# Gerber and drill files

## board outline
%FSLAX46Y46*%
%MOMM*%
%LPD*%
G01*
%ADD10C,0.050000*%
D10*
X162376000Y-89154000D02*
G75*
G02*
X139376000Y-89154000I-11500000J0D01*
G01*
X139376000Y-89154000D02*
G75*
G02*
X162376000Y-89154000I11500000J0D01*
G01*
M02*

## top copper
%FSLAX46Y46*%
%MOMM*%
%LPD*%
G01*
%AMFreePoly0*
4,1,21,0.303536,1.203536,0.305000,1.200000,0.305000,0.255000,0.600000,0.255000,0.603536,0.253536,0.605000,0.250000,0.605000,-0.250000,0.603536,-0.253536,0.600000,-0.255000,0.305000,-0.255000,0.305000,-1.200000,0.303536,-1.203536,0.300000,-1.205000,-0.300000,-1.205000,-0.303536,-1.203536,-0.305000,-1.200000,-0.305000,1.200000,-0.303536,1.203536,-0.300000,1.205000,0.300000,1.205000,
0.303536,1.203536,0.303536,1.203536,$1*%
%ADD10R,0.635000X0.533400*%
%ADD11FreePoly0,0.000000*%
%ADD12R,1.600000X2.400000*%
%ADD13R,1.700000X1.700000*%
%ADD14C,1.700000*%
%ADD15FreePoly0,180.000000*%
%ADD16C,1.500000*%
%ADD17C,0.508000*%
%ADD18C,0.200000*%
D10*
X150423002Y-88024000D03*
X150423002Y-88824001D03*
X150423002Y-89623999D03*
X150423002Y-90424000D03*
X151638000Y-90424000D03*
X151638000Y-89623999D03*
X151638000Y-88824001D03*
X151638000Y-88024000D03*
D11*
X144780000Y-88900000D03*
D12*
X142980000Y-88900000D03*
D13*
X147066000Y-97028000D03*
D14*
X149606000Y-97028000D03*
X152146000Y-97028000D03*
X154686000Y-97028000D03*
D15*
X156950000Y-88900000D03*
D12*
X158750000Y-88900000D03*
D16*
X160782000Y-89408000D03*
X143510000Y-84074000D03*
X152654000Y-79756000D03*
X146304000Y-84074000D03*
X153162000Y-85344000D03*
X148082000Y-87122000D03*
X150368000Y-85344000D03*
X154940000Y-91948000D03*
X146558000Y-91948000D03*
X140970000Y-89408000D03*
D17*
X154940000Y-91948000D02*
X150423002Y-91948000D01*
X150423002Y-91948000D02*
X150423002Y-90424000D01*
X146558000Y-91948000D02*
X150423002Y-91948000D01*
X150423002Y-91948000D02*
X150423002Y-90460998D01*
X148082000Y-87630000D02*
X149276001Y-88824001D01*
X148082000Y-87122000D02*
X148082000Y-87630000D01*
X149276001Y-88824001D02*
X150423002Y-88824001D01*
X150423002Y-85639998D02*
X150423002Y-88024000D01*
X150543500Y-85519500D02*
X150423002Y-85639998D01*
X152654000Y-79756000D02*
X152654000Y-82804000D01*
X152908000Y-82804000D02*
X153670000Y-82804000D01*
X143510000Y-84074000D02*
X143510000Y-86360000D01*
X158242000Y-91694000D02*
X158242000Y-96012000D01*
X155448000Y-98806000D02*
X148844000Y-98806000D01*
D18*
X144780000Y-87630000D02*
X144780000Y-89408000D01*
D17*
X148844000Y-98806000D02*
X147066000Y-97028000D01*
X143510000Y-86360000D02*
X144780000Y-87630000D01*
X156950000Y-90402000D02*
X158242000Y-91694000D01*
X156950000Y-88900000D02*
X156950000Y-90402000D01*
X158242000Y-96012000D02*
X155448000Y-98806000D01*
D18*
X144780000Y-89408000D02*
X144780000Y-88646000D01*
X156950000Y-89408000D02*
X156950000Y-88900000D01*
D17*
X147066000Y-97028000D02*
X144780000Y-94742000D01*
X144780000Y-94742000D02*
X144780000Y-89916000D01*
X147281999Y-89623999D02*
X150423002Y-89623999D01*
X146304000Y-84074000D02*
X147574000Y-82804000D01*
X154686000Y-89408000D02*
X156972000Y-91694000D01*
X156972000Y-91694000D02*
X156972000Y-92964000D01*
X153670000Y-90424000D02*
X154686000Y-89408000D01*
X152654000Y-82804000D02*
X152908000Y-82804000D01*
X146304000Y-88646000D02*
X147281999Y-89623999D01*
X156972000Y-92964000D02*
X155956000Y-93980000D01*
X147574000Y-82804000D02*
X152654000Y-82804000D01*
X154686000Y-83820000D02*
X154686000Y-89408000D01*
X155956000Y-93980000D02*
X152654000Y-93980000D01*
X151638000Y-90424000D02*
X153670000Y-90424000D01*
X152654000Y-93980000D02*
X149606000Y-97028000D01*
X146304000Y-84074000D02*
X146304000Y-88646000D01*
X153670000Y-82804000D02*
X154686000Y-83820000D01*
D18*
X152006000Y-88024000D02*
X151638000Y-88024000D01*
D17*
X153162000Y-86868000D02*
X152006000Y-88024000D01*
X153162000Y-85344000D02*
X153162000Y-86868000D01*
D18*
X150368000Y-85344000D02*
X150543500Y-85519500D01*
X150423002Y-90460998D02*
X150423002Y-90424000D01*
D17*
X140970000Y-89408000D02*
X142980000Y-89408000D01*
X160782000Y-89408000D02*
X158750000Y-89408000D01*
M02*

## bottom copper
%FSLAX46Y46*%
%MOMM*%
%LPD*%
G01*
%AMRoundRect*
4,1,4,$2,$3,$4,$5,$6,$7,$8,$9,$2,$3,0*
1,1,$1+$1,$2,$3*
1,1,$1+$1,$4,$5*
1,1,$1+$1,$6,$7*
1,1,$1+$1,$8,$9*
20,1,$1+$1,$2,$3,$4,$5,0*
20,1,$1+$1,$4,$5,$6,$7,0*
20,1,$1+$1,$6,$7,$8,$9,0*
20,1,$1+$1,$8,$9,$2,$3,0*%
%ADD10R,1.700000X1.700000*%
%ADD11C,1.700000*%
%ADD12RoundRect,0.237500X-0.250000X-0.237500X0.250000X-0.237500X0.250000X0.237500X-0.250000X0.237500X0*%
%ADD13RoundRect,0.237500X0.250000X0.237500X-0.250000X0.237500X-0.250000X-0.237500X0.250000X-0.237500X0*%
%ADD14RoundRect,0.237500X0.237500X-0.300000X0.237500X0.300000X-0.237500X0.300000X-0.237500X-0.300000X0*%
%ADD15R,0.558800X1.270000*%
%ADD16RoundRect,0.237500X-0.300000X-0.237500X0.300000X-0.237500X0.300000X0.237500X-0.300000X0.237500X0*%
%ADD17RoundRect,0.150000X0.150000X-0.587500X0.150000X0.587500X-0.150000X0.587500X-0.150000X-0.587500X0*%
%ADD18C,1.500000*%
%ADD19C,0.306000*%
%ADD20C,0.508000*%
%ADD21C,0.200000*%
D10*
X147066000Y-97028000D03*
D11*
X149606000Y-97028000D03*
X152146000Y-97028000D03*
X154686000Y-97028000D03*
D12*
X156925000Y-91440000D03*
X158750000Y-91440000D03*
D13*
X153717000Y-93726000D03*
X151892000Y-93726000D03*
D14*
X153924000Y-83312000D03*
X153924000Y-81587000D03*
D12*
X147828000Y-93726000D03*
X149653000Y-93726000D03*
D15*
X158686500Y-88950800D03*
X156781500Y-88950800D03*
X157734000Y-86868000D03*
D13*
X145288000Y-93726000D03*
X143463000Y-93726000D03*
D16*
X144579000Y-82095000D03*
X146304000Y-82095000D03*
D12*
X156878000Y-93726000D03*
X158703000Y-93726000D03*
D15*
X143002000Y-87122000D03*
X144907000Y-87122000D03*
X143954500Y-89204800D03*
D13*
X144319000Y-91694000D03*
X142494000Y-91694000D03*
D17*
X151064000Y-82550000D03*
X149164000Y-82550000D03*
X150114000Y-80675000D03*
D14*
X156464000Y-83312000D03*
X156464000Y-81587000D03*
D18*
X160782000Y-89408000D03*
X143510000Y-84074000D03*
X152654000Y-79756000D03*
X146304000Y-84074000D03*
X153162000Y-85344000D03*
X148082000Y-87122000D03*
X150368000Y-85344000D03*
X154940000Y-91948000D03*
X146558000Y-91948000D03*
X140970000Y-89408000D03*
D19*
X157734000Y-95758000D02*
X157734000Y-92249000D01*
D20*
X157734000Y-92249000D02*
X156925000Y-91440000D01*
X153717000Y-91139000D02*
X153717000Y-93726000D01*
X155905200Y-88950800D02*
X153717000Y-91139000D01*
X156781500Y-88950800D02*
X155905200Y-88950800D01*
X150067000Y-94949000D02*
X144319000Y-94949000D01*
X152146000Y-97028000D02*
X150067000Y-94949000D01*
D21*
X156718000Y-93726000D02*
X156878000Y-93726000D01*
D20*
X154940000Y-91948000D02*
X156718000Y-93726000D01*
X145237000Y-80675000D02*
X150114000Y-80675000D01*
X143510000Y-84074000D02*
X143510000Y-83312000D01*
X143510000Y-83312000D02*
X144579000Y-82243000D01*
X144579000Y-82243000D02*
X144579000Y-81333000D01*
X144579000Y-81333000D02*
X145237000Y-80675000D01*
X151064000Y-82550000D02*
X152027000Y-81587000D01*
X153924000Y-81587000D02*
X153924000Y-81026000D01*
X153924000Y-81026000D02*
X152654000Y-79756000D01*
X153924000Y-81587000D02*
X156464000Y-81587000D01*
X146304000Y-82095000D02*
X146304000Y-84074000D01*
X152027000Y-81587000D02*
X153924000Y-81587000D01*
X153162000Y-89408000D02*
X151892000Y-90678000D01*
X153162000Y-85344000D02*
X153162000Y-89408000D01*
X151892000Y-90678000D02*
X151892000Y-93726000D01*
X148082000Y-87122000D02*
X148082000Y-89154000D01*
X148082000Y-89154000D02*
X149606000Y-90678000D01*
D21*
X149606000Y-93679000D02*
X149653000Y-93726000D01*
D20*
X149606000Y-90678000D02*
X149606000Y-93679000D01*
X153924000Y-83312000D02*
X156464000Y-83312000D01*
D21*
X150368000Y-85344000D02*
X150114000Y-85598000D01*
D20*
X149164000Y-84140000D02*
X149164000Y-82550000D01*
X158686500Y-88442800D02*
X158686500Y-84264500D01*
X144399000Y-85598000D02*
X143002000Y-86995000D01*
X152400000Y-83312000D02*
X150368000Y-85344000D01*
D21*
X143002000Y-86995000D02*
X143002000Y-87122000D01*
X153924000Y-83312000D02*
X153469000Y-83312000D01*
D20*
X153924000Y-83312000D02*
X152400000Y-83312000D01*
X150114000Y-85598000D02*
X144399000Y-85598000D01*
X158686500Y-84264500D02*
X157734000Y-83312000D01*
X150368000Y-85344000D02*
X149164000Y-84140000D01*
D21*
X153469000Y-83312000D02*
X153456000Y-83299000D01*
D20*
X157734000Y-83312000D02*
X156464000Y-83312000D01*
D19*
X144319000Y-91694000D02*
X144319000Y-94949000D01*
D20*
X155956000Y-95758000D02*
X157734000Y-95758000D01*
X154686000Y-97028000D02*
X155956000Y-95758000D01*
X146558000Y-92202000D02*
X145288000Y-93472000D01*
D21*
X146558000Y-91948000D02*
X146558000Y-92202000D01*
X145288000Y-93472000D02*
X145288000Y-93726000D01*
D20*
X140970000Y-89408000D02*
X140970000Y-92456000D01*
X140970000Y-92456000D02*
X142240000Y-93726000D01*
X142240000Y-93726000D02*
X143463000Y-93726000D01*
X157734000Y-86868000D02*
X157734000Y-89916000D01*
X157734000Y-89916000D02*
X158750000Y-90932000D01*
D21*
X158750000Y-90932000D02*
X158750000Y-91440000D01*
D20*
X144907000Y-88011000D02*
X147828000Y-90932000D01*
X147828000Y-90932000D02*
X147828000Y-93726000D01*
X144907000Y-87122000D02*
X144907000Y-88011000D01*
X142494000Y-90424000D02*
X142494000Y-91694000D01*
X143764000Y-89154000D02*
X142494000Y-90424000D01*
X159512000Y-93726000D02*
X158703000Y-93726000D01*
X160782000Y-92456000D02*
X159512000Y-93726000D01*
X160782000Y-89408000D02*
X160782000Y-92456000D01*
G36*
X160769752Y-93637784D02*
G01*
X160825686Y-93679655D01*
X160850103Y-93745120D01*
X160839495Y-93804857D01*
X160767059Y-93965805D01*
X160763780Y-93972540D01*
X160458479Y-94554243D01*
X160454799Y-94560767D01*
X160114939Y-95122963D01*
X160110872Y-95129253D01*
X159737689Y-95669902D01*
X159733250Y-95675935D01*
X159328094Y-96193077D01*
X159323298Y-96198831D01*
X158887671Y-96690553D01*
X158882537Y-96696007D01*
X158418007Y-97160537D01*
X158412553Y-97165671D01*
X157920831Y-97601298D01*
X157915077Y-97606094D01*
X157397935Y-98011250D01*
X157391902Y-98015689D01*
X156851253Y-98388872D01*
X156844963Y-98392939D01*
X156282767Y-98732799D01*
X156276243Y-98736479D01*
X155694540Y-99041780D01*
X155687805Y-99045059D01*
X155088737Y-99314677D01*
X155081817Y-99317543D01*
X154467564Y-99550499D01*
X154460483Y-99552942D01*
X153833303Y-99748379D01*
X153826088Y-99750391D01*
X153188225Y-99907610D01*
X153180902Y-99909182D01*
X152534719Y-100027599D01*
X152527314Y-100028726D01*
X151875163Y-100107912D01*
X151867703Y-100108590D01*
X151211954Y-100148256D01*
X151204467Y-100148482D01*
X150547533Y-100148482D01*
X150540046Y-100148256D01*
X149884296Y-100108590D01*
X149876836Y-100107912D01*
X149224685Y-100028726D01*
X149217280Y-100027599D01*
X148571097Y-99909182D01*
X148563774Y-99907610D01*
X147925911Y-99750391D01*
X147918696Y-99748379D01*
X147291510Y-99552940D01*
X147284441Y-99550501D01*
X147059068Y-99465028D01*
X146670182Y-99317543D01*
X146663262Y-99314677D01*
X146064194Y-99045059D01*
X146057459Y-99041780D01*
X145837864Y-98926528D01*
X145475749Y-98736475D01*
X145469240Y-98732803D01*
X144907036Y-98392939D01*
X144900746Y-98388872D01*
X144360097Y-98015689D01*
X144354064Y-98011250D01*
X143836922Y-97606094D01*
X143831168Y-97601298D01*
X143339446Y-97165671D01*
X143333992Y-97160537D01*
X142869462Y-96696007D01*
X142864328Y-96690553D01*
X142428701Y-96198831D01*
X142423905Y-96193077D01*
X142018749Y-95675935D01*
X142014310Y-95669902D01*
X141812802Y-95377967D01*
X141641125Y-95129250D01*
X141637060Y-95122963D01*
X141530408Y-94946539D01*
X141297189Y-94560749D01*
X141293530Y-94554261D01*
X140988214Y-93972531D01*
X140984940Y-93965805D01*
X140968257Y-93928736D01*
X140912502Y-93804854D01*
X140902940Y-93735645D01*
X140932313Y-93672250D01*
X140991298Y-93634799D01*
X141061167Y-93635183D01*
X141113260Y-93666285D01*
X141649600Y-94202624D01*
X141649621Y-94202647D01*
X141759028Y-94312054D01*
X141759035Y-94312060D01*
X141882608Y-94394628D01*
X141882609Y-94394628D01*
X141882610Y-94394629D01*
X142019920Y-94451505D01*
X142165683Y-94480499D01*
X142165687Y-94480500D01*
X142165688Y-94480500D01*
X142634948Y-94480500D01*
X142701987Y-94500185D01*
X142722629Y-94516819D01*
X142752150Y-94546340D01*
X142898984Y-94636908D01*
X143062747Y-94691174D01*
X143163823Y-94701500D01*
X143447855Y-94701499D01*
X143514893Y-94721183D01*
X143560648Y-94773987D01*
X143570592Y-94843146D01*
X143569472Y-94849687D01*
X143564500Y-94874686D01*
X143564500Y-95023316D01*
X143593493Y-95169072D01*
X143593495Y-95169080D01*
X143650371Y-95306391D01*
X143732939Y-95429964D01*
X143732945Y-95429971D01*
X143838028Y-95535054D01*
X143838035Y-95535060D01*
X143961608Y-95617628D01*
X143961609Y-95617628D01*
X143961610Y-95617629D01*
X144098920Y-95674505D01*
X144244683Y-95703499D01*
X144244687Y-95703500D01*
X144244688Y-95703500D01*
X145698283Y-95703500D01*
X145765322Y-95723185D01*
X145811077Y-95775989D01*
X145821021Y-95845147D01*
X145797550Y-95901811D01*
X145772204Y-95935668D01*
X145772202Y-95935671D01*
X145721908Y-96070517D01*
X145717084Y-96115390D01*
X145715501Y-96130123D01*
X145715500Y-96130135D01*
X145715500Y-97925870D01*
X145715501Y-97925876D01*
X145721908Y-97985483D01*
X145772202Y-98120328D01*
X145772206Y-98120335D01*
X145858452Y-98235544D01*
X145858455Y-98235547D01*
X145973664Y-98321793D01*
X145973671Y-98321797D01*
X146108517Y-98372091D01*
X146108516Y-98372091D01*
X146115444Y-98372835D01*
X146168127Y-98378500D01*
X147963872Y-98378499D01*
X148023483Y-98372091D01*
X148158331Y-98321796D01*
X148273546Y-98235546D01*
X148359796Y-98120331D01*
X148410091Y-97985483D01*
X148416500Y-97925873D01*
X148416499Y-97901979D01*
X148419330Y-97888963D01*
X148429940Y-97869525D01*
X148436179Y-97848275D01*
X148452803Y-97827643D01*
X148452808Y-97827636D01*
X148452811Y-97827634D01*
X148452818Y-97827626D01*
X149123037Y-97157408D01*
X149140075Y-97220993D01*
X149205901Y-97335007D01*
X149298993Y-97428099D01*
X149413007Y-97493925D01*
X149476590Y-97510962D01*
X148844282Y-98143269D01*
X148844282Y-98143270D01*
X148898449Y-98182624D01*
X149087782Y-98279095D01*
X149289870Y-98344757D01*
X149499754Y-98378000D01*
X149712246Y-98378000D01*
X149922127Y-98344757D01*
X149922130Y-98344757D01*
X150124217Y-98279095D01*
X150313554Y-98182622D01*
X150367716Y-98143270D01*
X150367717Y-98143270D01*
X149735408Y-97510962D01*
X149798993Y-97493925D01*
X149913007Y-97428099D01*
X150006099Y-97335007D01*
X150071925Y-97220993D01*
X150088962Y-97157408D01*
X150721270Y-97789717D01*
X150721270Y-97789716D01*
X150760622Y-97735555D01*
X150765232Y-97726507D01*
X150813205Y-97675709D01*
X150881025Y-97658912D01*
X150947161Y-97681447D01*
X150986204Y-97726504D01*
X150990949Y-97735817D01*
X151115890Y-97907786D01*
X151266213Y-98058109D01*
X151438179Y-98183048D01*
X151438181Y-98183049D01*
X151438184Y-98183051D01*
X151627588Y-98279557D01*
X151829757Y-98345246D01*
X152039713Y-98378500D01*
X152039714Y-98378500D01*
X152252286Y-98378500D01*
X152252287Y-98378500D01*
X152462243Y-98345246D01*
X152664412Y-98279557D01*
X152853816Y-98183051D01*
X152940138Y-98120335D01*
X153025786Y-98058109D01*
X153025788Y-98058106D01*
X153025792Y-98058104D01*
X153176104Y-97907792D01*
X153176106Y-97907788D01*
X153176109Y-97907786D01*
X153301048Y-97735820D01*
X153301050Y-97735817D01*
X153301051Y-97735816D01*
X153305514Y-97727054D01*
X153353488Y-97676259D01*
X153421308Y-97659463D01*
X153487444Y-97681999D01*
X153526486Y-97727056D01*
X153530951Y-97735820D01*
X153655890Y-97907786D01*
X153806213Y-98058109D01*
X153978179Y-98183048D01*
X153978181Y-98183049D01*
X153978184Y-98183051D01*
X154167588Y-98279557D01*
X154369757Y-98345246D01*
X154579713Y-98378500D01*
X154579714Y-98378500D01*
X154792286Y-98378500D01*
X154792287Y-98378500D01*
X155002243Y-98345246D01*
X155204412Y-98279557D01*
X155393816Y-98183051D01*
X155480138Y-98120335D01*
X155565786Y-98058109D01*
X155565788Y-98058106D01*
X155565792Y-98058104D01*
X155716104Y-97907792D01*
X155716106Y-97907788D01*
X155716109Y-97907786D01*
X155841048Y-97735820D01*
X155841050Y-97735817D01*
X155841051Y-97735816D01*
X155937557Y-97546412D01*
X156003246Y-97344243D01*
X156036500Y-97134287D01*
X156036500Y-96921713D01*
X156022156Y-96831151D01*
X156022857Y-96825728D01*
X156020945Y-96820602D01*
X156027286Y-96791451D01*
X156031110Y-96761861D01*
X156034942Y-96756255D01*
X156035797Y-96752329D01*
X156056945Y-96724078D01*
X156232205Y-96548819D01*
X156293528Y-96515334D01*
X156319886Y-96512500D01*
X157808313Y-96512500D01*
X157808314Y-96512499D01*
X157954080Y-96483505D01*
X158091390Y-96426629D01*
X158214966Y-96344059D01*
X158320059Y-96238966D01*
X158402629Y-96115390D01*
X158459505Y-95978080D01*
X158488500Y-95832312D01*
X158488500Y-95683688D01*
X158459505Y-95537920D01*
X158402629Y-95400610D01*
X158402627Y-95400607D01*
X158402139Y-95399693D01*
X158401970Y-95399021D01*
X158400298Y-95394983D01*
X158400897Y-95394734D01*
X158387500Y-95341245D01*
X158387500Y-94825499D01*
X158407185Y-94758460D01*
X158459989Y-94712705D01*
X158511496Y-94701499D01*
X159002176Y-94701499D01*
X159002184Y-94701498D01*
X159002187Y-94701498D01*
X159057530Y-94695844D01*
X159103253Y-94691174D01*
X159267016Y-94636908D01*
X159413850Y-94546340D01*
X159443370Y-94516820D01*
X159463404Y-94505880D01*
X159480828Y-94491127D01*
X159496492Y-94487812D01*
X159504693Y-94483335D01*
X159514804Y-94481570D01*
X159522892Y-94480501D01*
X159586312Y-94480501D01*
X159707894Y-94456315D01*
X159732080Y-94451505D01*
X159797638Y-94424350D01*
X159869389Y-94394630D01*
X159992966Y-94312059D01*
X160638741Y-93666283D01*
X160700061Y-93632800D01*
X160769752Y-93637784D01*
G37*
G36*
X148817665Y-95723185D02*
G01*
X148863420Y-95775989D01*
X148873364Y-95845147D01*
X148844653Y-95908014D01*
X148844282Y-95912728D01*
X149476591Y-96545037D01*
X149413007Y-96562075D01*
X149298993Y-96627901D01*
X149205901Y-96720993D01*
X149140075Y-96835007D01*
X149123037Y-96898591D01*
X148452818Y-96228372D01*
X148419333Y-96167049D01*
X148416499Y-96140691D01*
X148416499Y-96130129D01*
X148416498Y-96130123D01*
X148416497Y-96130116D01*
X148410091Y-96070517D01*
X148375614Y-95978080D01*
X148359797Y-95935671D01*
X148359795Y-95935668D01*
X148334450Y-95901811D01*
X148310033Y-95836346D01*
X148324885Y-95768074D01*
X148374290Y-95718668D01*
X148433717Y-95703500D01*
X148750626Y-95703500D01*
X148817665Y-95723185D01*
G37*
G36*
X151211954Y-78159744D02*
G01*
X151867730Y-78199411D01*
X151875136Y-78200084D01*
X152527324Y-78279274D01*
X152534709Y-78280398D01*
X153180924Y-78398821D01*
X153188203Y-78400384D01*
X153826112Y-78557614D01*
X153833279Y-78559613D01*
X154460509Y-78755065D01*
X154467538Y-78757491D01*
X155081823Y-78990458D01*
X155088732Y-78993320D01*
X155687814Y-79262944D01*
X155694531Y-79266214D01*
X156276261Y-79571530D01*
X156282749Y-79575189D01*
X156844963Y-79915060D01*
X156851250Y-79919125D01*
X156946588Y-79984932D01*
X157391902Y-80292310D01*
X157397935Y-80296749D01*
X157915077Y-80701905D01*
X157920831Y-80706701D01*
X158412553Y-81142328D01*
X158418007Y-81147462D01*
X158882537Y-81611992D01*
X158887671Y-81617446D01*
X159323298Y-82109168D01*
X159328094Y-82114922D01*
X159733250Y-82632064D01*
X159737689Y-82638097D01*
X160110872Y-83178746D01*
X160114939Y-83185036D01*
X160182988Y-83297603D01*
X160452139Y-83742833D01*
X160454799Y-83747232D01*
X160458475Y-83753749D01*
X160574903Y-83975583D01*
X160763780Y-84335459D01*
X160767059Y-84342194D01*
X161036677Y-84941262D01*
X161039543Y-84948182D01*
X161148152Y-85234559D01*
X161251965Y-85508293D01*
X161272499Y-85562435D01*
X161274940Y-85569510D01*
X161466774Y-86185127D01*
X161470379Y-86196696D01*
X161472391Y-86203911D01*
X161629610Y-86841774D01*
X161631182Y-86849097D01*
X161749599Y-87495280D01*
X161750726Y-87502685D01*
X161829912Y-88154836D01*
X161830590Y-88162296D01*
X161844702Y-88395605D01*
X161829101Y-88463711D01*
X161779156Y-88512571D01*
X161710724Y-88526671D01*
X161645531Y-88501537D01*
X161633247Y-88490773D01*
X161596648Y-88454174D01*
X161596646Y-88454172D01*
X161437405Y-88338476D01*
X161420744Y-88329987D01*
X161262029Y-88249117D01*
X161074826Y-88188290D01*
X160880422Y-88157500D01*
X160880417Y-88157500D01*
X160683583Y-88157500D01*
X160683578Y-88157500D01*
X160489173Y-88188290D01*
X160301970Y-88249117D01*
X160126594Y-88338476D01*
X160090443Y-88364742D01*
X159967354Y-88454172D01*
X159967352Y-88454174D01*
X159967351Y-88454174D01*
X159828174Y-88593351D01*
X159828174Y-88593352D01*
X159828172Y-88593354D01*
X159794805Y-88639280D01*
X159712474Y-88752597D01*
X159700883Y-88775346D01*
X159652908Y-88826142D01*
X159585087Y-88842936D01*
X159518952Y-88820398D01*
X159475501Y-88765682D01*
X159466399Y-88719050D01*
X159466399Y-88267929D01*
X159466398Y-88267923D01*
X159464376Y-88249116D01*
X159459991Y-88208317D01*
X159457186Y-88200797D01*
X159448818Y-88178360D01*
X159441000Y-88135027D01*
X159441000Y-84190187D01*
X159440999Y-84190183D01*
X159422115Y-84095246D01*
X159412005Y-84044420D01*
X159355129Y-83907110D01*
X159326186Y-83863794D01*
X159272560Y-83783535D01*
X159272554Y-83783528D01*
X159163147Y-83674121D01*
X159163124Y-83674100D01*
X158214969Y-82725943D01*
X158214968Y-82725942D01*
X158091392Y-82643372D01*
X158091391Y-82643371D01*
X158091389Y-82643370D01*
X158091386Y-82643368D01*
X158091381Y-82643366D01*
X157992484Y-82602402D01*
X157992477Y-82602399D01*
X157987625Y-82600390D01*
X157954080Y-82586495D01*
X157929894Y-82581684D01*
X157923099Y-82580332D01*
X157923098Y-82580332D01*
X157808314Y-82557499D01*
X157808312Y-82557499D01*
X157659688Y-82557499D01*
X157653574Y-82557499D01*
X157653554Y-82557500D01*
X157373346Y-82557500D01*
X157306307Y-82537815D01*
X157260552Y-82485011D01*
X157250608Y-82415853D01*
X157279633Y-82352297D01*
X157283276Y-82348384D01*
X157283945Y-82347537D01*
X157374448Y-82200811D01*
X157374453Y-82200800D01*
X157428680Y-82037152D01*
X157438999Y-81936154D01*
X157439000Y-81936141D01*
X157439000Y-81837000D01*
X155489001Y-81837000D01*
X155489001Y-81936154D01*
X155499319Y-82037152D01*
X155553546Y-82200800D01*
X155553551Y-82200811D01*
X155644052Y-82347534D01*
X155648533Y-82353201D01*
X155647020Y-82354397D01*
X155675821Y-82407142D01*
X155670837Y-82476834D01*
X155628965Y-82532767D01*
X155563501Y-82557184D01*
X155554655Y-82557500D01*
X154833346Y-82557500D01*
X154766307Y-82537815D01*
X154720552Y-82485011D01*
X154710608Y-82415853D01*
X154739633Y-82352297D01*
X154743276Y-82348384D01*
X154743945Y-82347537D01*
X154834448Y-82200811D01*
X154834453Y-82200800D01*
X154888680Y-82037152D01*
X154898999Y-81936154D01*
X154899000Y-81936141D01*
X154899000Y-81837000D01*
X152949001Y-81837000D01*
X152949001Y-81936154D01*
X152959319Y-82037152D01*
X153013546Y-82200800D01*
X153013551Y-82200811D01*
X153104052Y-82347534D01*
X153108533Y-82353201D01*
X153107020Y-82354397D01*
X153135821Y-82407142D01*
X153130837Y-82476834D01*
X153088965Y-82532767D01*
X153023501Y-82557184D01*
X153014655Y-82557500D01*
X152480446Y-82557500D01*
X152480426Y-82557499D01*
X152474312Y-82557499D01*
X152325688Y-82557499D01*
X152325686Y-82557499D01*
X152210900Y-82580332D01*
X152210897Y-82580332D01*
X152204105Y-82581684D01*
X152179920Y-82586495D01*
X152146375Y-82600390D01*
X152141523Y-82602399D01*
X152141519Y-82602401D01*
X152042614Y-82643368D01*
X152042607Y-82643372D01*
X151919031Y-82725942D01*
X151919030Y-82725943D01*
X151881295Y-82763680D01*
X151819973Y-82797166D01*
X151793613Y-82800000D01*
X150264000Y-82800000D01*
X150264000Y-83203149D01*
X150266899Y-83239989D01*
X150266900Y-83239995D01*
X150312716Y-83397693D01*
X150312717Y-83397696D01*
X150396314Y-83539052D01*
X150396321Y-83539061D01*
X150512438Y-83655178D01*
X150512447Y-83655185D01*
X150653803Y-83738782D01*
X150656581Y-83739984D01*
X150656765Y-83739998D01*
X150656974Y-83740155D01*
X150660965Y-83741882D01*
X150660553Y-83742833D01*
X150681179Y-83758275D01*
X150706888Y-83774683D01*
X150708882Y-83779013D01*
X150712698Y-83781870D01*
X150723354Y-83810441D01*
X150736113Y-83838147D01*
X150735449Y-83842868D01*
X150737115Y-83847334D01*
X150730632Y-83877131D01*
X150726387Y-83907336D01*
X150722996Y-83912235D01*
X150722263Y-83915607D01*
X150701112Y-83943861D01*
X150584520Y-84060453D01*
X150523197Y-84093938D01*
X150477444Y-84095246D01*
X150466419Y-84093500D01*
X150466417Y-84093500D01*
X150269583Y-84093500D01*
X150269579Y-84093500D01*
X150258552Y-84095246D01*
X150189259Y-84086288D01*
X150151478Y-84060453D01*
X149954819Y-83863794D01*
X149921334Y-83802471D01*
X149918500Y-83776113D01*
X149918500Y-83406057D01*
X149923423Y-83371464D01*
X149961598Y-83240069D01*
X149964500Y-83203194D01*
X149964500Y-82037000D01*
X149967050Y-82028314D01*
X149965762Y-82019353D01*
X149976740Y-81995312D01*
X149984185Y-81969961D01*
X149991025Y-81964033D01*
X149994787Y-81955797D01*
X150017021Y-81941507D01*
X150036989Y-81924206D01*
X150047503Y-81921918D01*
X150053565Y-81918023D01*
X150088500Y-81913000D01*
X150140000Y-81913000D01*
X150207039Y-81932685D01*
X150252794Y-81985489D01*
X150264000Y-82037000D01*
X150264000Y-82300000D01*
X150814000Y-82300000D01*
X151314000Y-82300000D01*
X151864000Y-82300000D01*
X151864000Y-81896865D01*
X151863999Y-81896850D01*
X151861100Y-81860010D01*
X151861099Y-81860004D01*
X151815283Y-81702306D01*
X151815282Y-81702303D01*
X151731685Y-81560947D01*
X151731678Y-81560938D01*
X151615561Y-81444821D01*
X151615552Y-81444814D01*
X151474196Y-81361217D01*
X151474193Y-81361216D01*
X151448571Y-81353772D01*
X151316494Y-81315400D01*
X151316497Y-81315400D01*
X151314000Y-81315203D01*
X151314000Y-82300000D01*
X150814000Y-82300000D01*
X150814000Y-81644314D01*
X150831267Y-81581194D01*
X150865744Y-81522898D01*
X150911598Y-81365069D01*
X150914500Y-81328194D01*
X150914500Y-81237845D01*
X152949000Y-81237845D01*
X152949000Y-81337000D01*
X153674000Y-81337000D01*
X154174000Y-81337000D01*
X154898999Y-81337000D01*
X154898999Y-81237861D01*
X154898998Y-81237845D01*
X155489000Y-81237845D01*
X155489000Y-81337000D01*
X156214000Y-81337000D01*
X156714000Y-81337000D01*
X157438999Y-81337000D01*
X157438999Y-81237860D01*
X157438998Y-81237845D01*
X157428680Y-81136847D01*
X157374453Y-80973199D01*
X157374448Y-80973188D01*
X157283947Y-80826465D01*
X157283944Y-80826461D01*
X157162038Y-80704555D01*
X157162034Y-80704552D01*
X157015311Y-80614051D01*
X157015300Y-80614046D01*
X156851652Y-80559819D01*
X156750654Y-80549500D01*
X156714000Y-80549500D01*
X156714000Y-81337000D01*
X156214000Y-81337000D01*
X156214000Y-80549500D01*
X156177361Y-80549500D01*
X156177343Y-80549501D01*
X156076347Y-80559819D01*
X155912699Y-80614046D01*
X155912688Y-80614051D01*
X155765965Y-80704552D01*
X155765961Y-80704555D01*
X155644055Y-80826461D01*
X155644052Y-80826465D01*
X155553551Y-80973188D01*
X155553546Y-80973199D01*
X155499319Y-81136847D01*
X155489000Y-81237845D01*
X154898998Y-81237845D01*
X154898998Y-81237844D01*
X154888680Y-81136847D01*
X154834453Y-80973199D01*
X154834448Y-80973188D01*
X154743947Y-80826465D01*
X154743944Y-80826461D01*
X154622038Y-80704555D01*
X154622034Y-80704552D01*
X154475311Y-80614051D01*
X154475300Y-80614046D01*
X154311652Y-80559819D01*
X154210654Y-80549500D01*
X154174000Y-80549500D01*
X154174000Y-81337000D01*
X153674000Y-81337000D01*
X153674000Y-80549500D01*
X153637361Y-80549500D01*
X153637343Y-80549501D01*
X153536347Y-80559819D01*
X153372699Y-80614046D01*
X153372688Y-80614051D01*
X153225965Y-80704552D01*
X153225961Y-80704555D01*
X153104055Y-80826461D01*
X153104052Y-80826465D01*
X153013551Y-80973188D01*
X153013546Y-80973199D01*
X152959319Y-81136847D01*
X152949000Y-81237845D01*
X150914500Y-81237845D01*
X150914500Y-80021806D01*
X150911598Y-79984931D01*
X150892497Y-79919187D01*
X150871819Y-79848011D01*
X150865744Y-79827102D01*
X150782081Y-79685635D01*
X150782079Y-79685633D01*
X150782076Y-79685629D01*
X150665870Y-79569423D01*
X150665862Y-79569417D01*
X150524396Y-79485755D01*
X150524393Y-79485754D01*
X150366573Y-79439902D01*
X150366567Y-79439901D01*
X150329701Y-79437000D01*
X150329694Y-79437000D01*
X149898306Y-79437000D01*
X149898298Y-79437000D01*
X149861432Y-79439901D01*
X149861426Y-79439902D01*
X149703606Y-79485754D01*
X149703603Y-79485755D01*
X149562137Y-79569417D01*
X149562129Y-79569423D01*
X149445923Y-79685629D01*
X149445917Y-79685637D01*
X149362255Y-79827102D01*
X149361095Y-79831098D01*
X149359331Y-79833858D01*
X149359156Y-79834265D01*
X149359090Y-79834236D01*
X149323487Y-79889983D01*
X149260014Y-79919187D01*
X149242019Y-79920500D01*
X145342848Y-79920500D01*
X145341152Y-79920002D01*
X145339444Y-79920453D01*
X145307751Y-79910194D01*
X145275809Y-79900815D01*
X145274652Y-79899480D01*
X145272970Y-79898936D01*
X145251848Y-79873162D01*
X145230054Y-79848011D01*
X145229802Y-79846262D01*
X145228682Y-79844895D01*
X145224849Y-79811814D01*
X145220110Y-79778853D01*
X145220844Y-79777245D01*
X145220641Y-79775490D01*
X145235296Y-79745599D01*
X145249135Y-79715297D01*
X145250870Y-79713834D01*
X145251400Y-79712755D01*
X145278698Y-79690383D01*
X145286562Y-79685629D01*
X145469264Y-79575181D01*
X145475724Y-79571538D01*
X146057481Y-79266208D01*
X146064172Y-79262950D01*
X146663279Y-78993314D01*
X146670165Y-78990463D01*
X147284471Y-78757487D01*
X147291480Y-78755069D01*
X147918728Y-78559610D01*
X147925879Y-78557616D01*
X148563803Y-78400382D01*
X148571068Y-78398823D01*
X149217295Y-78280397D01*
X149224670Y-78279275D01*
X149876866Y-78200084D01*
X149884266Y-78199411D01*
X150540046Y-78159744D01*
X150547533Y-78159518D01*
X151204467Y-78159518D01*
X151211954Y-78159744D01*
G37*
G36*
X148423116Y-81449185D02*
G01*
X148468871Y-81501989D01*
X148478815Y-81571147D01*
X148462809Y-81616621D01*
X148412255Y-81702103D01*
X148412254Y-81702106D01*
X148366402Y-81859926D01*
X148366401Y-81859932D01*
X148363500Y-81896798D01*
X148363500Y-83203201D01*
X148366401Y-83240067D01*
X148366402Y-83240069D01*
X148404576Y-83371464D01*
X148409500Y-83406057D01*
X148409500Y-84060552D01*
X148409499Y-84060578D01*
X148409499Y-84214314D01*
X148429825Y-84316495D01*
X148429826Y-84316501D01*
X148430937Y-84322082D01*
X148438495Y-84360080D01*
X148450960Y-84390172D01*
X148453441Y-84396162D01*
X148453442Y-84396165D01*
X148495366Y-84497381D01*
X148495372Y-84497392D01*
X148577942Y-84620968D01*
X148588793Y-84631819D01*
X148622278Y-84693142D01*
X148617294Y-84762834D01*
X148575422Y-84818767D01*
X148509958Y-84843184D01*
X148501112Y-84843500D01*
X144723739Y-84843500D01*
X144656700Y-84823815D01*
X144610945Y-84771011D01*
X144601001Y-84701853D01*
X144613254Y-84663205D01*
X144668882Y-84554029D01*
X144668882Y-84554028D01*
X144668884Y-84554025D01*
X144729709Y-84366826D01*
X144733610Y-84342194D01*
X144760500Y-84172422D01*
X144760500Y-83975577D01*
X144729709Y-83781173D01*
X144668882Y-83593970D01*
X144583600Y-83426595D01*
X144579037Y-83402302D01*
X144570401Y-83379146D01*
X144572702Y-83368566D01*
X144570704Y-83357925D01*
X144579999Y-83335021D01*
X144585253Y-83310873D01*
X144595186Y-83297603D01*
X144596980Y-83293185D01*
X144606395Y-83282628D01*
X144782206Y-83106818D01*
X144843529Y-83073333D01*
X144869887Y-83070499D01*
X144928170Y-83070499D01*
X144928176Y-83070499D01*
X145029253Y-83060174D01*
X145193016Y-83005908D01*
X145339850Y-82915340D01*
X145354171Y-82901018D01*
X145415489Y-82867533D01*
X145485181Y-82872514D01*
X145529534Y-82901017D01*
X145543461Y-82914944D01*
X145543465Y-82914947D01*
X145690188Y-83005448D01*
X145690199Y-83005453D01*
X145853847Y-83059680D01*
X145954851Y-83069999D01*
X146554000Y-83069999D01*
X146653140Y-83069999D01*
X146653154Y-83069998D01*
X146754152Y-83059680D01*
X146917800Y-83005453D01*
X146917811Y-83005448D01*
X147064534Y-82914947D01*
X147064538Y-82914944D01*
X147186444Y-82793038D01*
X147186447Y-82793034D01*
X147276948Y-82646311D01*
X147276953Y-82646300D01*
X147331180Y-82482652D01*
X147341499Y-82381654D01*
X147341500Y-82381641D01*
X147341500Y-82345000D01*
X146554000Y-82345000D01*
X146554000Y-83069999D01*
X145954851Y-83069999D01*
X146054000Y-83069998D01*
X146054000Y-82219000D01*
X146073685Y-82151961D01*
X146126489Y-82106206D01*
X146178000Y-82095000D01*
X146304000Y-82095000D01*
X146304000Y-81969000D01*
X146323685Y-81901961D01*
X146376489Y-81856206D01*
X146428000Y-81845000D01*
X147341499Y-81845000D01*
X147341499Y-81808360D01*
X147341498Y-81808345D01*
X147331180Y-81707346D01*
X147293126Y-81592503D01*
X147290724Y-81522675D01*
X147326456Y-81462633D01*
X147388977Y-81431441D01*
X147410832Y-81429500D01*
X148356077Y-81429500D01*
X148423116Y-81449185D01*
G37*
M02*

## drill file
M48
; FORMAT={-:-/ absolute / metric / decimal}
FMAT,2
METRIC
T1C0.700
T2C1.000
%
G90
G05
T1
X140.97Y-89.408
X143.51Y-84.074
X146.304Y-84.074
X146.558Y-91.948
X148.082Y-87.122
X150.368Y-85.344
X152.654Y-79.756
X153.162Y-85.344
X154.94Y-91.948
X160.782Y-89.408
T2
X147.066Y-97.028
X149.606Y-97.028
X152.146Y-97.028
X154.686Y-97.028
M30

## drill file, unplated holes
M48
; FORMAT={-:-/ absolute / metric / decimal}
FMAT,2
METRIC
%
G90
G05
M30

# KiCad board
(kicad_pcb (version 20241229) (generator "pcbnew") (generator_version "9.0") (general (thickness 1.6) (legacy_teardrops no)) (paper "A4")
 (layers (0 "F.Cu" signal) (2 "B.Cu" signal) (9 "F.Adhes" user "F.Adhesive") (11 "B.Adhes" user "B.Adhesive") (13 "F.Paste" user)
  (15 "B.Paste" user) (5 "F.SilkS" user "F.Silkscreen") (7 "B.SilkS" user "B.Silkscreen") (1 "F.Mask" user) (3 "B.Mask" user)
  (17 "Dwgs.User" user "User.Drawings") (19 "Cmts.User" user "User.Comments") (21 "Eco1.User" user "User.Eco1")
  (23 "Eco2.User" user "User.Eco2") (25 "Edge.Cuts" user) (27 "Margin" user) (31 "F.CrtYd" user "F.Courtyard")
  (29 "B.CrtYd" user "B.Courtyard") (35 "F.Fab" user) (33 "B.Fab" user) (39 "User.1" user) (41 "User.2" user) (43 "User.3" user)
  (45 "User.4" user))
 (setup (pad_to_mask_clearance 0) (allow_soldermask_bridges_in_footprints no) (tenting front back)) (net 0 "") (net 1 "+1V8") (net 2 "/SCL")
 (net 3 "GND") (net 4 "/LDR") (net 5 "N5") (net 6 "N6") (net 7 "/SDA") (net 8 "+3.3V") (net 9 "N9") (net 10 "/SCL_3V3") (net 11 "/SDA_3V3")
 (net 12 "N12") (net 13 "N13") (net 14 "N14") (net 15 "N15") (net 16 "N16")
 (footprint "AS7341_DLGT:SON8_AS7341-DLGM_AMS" (layer "F.Cu") (at 151.030501 89.224)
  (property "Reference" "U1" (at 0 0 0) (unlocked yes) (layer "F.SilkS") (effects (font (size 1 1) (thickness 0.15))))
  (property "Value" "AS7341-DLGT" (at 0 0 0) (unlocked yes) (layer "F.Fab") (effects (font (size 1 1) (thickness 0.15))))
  (pad "1" smd rect (at -0.607499 -1.2) (size 0.635 0.5334) (layers "F.Cu" "F.Mask" "F.Paste") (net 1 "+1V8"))
  (pad "2" smd rect (at -0.607499 -0.399999) (size 0.635 0.5334) (layers "F.Cu" "F.Mask" "F.Paste") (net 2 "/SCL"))
  (pad "3" smd rect (at -0.607499 0.399999) (size 0.635 0.5334) (layers "F.Cu" "F.Mask" "F.Paste") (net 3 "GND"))
  (pad "4" smd rect (at -0.607499 1.2) (size 0.635 0.5334) (layers "F.Cu" "F.Mask" "F.Paste") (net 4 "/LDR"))
  (pad "5" smd rect (at 0.607499 1.2) (size 0.635 0.5334) (layers "F.Cu" "F.Mask" "F.Paste") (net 3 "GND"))
  (pad "6" smd rect (at 0.607499 0.399999) (size 0.635 0.5334) (layers "F.Cu" "F.Mask" "F.Paste") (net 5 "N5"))
  (pad "7" smd rect (at 0.607499 -0.399999) (size 0.635 0.5334) (layers "F.Cu" "F.Mask" "F.Paste") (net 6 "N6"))
  (pad "8" smd rect (at 0.607499 -1.2) (size 0.635 0.5334) (layers "F.Cu" "F.Mask" "F.Paste") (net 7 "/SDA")))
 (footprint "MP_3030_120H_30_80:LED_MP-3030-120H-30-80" (layer "F.Cu") (at 143.78 88.9)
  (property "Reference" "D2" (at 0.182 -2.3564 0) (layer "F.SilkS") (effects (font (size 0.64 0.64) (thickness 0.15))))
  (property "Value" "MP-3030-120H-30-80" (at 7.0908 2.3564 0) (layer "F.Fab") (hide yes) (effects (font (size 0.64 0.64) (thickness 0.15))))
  (pad "A" smd custom (at 1 0) (size 0.4 0.4) (layers "F.Cu") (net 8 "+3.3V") (options (clearance outline) (anchor rect)) (primitives))
  (pad "C" smd rect (at -0.8 0) (size 1.6 2.4) (layers "F.Cu" "F.Mask" "F.Paste") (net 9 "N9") (solder_mask_margin 0.102)))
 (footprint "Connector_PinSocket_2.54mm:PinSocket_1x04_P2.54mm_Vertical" (layer "F.Cu") (at 147.066 97.028 90)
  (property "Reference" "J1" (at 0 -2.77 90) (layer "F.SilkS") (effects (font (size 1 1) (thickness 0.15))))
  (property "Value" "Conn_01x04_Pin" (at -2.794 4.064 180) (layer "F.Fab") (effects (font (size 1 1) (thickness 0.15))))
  (pad "1" thru_hole rect (at 0 0 90) (size 1.7 1.7) (drill 1) (layers "*.Cu" "*.Mask") (remove_unused_layers no) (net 8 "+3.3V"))
  (pad "2" thru_hole circle (at 0 2.54 90) (size 1.7 1.7) (drill 1) (layers "*.Cu" "*.Mask") (remove_unused_layers no) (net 3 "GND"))
  (pad "3" thru_hole circle (at 0 5.08 90) (size 1.7 1.7) (drill 1) (layers "*.Cu" "*.Mask") (remove_unused_layers no) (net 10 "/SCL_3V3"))
  (pad "4" thru_hole circle (at 0 7.62 90) (size 1.7 1.7) (drill 1) (layers "*.Cu" "*.Mask") (remove_unused_layers no) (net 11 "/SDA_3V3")))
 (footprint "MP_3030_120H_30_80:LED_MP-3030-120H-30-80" (layer "F.Cu") (at 157.95 88.9 180)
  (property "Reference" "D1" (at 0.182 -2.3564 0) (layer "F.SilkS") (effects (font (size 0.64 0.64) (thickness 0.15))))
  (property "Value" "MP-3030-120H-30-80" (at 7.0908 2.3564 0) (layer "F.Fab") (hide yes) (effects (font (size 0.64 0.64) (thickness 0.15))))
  (pad "A" smd custom (at 1 0 180) (size 0.4 0.4) (layers "F.Cu") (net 8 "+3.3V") (options (clearance outline) (anchor rect)) (primitives))
  (pad "C" smd rect (at -0.8 0 180) (size 1.6 2.4) (layers "F.Cu" "F.Mask" "F.Paste") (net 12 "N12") (solder_mask_margin 0.102)))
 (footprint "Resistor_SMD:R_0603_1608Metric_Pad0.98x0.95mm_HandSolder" (layer "B.Cu") (at 157.8375 91.44)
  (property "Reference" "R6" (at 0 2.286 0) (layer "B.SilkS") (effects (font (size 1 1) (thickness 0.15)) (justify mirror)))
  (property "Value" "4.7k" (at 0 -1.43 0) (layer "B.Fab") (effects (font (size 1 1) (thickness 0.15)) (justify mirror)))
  (pad "1" smd roundrect (at -0.9125 0) (size 0.975 0.95) (layers "B.Cu" "B.Mask" "B.Paste") (roundrect_rratio 0.25) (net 11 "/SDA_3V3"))
  (pad "2" smd roundrect (at 0.9125 0) (size 0.975 0.95) (layers "B.Cu" "B.Mask" "B.Paste") (roundrect_rratio 0.25) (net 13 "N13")))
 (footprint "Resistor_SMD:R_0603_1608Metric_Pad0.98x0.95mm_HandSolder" (layer "B.Cu") (at 152.8045 93.726 180)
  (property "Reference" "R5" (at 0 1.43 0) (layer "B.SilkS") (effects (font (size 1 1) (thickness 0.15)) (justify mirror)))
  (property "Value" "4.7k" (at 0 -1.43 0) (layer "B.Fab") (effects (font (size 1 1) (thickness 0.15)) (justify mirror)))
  (pad "1" smd roundrect (at -0.9125 0 180) (size 0.975 0.95) (layers "B.Cu" "B.Mask" "B.Paste") (roundrect_rratio 0.25) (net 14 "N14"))
  (pad "2" smd roundrect (at 0.9125 0 180) (size 0.975 0.95) (layers "B.Cu" "B.Mask" "B.Paste") (roundrect_rratio 0.25) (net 7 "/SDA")))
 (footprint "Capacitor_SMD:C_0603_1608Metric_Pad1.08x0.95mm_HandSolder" (layer "B.Cu") (at 153.924 82.4495 90)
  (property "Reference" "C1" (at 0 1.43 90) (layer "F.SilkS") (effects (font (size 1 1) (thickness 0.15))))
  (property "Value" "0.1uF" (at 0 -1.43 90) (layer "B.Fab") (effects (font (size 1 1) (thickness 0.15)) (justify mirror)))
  (pad "1" smd roundrect (at -0.8625 0 90) (size 1.075 0.95) (layers "B.Cu" "B.Mask" "B.Paste") (roundrect_rratio 0.25) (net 1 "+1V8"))
  (pad "2" smd roundrect (at 0.8625 0 90) (size 1.075 0.95) (layers "B.Cu" "B.Mask" "B.Paste") (roundrect_rratio 0.25) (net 3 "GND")))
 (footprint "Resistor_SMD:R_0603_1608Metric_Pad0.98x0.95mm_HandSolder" (layer "B.Cu") (at 148.7405 93.726)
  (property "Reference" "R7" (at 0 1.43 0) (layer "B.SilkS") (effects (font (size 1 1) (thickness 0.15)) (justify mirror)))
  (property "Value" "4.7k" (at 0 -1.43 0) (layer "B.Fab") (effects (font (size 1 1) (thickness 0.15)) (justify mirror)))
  (pad "1" smd roundrect (at -0.9125 0) (size 0.975 0.95) (layers "B.Cu" "B.Mask" "B.Paste") (roundrect_rratio 0.25) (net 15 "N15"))
  (pad "2" smd roundrect (at 0.9125 0) (size 0.975 0.95) (layers "B.Cu" "B.Mask" "B.Paste") (roundrect_rratio 0.25) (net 2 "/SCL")))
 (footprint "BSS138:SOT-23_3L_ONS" (layer "B.Cu") (at 157.734 87.9094 180)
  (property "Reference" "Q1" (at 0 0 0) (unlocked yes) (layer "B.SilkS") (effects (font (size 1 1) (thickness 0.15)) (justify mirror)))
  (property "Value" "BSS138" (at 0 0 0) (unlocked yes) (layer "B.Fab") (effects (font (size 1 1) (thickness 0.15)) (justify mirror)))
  (pad "1" smd rect (at -0.9525 -1.0414 180) (size 0.5588 1.27) (layers "B.Cu" "B.Mask" "B.Paste") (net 1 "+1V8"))
  (pad "2" smd rect (at 0.9525 -1.0414 180) (size 0.5588 1.27) (layers "B.Cu" "B.Mask" "B.Paste") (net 14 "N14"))
  (pad "3" smd rect (at 0 1.0414 180) (size 0.5588 1.27) (layers "B.Cu" "B.Mask" "B.Paste") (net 13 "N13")))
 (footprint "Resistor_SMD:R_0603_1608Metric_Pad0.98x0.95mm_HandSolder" (layer "B.Cu") (at 144.3755 93.726 180)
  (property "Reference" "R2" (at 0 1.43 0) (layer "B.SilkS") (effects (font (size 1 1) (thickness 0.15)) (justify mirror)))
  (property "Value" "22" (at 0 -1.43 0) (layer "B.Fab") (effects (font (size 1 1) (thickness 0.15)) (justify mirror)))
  (pad "1" smd roundrect (at -0.9125 0 180) (size 0.975 0.95) (layers "B.Cu" "B.Mask" "B.Paste") (roundrect_rratio 0.25) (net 4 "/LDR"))
  (pad "2" smd roundrect (at 0.9125 0 180) (size 0.975 0.95) (layers "B.Cu" "B.Mask" "B.Paste") (roundrect_rratio 0.25) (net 9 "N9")))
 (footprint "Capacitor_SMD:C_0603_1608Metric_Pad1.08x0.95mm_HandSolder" (layer "B.Cu") (at 145.4415 82.095)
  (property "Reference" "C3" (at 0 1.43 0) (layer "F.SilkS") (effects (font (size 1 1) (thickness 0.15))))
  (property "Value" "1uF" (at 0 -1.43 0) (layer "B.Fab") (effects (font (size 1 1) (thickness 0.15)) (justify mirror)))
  (pad "1" smd roundrect (at -0.8625 0) (size 1.075 0.95) (layers "B.Cu" "B.Mask" "B.Paste") (roundrect_rratio 0.25) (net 8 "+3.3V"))
  (pad "2" smd roundrect (at 0.8625 0) (size 1.075 0.95) (layers "B.Cu" "B.Mask" "B.Paste") (roundrect_rratio 0.25) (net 3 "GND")))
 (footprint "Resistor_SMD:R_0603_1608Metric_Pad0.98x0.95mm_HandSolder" (layer "B.Cu") (at 157.7905 93.726)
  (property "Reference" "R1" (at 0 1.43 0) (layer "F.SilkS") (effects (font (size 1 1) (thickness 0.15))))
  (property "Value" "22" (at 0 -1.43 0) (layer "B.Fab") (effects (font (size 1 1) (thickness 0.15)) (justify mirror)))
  (pad "1" smd roundrect (at -0.9125 0) (size 0.975 0.95) (layers "B.Cu" "B.Mask" "B.Paste") (roundrect_rratio 0.25) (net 4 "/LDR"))
  (pad "2" smd roundrect (at 0.9125 0) (size 0.975 0.95) (layers "B.Cu" "B.Mask" "B.Paste") (roundrect_rratio 0.25) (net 12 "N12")))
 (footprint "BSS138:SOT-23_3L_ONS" (layer "B.Cu") (at 143.9545 88.1634)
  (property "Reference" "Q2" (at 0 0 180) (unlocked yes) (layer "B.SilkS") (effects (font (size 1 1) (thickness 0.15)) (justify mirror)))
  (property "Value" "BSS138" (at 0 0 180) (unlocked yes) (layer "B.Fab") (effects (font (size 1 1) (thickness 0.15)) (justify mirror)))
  (pad "1" smd rect (at -0.9525 -1.0414) (size 0.5588 1.27) (layers "B.Cu" "B.Mask" "B.Paste") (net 1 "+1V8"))
  (pad "2" smd rect (at 0.9525 -1.0414) (size 0.5588 1.27) (layers "B.Cu" "B.Mask" "B.Paste") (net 15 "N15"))
  (pad "3" smd rect (at 0 1.0414) (size 0.5588 1.27) (layers "B.Cu" "B.Mask" "B.Paste") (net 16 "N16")))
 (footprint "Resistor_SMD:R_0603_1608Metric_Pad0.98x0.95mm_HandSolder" (layer "B.Cu") (at 143.4065 91.694 180)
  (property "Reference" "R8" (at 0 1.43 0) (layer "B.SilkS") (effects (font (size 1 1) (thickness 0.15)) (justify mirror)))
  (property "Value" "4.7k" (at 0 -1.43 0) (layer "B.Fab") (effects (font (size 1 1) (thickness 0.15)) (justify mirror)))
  (pad "1" smd roundrect (at -0.9125 0 180) (size 0.975 0.95) (layers "B.Cu" "B.Mask" "B.Paste") (roundrect_rratio 0.25) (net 10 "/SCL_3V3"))
  (pad "2" smd roundrect (at 0.9125 0 180) (size 0.975 0.95) (layers "B.Cu" "B.Mask" "B.Paste") (roundrect_rratio 0.25) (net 16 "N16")))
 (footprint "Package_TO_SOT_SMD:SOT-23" (layer "B.Cu") (at 150.114 81.6125 90)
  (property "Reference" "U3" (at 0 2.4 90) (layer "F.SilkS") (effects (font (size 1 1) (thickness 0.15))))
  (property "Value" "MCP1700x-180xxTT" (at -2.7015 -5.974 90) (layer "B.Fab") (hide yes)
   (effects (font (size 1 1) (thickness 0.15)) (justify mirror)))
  (pad "1" smd roundrect (at -0.9375 0.95 90) (size 1.475 0.6) (layers "B.Cu" "B.Mask" "B.Paste") (roundrect_rratio 0.25) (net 3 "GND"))
  (pad "2" smd roundrect (at -0.9375 -0.95 90) (size 1.475 0.6) (layers "B.Cu" "B.Mask" "B.Paste") (roundrect_rratio 0.25) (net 1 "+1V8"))
  (pad "3" smd roundrect (at 0.9375 0 90) (size 1.475 0.6) (layers "B.Cu" "B.Mask" "B.Paste") (roundrect_rratio 0.25) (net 8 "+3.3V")))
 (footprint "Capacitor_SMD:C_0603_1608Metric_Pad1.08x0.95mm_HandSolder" (layer "B.Cu") (at 156.464 82.4495 90)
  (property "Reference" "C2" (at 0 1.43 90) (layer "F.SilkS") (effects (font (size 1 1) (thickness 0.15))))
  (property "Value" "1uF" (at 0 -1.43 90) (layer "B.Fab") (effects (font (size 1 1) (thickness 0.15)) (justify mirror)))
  (pad "1" smd roundrect (at -0.8625 0 90) (size 1.075 0.95) (layers "B.Cu" "B.Mask" "B.Paste") (roundrect_rratio 0.25) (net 1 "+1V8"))
  (pad "2" smd roundrect (at 0.8625 0 90) (size 1.075 0.95) (layers "B.Cu" "B.Mask" "B.Paste") (roundrect_rratio 0.25) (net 3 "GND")))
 (gr_circle (center 150.876 89.154) (end 162.376 89.154) (stroke (width 0.05) (type solid)) (fill no) (layer "Edge.Cuts"))
 (segment (start 143.51 84.074) (end 143.51 86.36) (width 0.508) (layer "F.Cu") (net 8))
 (segment (start 158.242 91.694) (end 158.242 96.012) (width 0.508) (layer "F.Cu") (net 8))
 (segment (start 155.448 98.806) (end 148.844 98.806) (width 0.508) (layer "F.Cu") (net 8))
 (segment (start 144.78 87.63) (end 144.78 89.408) (width 0.2) (layer "F.Cu") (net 8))
 (segment (start 148.844 98.806) (end 147.066 97.028) (width 0.508) (layer "F.Cu") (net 8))
 (segment (start 143.51 86.36) (end 144.78 87.63) (width 0.508) (layer "F.Cu") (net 8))
 (segment (start 156.95 90.402) (end 158.242 91.694) (width 0.508) (layer "F.Cu") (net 8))
 (segment (start 156.95 88.9) (end 156.95 90.402) (width 0.508) (layer "F.Cu") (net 8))
 (segment (start 158.242 96.012) (end 155.448 98.806) (width 0.508) (layer "F.Cu") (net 8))
 (segment (start 144.78 89.408) (end 144.78 88.646) (width 0.2) (layer "F.Cu") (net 8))
 (segment (start 156.95 89.408) (end 156.95 88.9) (width 0.2) (layer "F.Cu") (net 8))
 (segment (start 147.066 97.028) (end 144.78 94.742) (width 0.508) (layer "F.Cu") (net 8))
 (segment (start 144.78 94.742) (end 144.78 89.916) (width 0.508) (layer "F.Cu") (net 8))
 (via (at 143.51 84.074) (size 1.5) (drill 0.7) (layers "F.Cu" "B.Cu") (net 8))
 (segment (start 145.237 80.675) (end 150.114 80.675) (width 0.508) (layer "B.Cu") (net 8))
 (segment (start 143.51 84.074) (end 143.51 83.312) (width 0.508) (layer "B.Cu") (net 8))
 (segment (start 143.51 83.312) (end 144.579 82.243) (width 0.508) (layer "B.Cu") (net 8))
 (segment (start 144.579 82.243) (end 144.579 81.333) (width 0.508) (layer "B.Cu") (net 8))
 (segment (start 144.579 81.333) (end 145.237 80.675) (width 0.508) (layer "B.Cu") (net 8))
 (segment (start 147.281999 89.623999) (end 150.423002 89.623999) (width 0.508) (layer "F.Cu") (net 3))
 (segment (start 146.304 84.074) (end 147.574 82.804) (width 0.508) (layer "F.Cu") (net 3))
 (segment (start 154.686 89.408) (end 156.972 91.694) (width 0.508) (layer "F.Cu") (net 3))
 (segment (start 156.972 91.694) (end 156.972 92.964) (width 0.508) (layer "F.Cu") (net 3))
 (segment (start 153.67 90.424) (end 154.686 89.408) (width 0.508) (layer "F.Cu") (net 3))
 (segment (start 152.654 82.804) (end 152.908 82.804) (width 0.508) (layer "F.Cu") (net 3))
 (segment (start 146.304 88.646) (end 147.281999 89.623999) (width 0.508) (layer "F.Cu") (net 3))
 (segment (start 156.972 92.964) (end 155.956 93.98) (width 0.508) (layer "F.Cu") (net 3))
 (segment (start 152.654 79.756) (end 152.654 82.804) (width 0.508) (layer "F.Cu") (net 3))
 (segment (start 152.908 82.804) (end 153.67 82.804) (width 0.508) (layer "F.Cu") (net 3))
 (segment (start 147.574 82.804) (end 152.654 82.804) (width 0.508) (layer "F.Cu") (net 3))
 (segment (start 154.686 83.82) (end 154.686 89.408) (width 0.508) (layer "F.Cu") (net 3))
 (segment (start 155.956 93.98) (end 152.654 93.98) (width 0.508) (layer "F.Cu") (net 3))
 (segment (start 151.638 90.424) (end 153.67 90.424) (width 0.508) (layer "F.Cu") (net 3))
 (segment (start 152.654 93.98) (end 149.606 97.028) (width 0.508) (layer "F.Cu") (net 3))
 (segment (start 146.304 84.074) (end 146.304 88.646) (width 0.508) (layer "F.Cu") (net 3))
 (segment (start 153.67 82.804) (end 154.686 83.82) (width 0.508) (layer "F.Cu") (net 3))
 (via (at 152.654 79.756) (size 1.5) (drill 0.7) (layers "F.Cu" "B.Cu") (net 3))
 (via (at 146.304 84.074) (size 1.5) (drill 0.7) (layers "F.Cu" "B.Cu") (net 3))
 (segment (start 151.064 82.55) (end 152.027 81.587) (width 0.508) (layer "B.Cu") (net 3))
 (segment (start 153.924 81.587) (end 153.924 81.026) (width 0.508) (layer "B.Cu") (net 3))
 (segment (start 153.924 81.026) (end 152.654 79.756) (width 0.508) (layer "B.Cu") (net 3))
 (segment (start 153.924 81.587) (end 156.464 81.587) (width 0.508) (layer "B.Cu") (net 3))
 (segment (start 146.304 82.095) (end 146.304 84.074) (width 0.508) (layer "B.Cu") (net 3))
 (segment (start 152.027 81.587) (end 153.924 81.587) (width 0.508) (layer "B.Cu") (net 3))
 (segment (start 152.006 88.024) (end 151.638 88.024) (width 0.2) (layer "F.Cu") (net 7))
 (segment (start 153.162 86.868) (end 152.006 88.024) (width 0.508) (layer "F.Cu") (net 7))
 (segment (start 153.162 85.344) (end 153.162 86.868) (width 0.508) (layer "F.Cu") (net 7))
 (via (at 153.162 85.344) (size 1.5) (drill 0.7) (layers "F.Cu" "B.Cu") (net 7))
 (segment (start 153.162 89.408) (end 151.892 90.678) (width 0.508) (layer "B.Cu") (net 7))
 (segment (start 153.162 85.344) (end 153.162 89.408) (width 0.508) (layer "B.Cu") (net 7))
 (segment (start 151.892 90.678) (end 151.892 93.726) (width 0.508) (layer "B.Cu") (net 7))
 (segment (start 148.082 87.122) (end 148.082 87.63) (width 0.508) (layer "F.Cu") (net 2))
 (segment (start 148.082 87.63) (end 149.276001 88.824001) (width 0.508) (layer "F.Cu") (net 2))
 (segment (start 149.276001 88.824001) (end 150.423002 88.824001) (width 0.508) (layer "F.Cu") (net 2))
 (via (at 148.082 87.122) (size 1.5) (drill 0.7) (layers "F.Cu" "B.Cu") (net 2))
 (segment (start 148.082 87.122) (end 148.082 89.154) (width 0.508) (layer "B.Cu") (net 2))
 (segment (start 148.082 89.154) (end 149.606 90.678) (width 0.508) (layer "B.Cu") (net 2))
 (segment (start 149.606 93.679) (end 149.653 93.726) (width 0.2) (layer "B.Cu") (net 2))
 (segment (start 149.606 90.678) (end 149.606 93.679) (width 0.508) (layer "B.Cu") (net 2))
 (segment (start 150.423002 85.639998) (end 150.423002 88.024) (width 0.508) (layer "F.Cu") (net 1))
 (segment (start 150.368 85.344) (end 150.5435 85.5195) (width 0.2) (layer "F.Cu") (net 1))
 (segment (start 150.5435 85.5195) (end 150.423002 85.639998) (width 0.508) (layer "F.Cu") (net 1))
 (via (at 150.368 85.344) (size 1.5) (drill 0.7) (layers "F.Cu" "B.Cu") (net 1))
 (segment (start 153.924 83.312) (end 156.464 83.312) (width 0.508) (layer "B.Cu") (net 1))
 (segment (start 150.368 85.344) (end 150.114 85.598) (width 0.2) (layer "B.Cu") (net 1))
 (segment (start 149.164 84.14) (end 149.164 82.55) (width 0.508) (layer "B.Cu") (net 1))
 (segment (start 158.6865 88.4428) (end 158.6865 84.2645) (width 0.508) (layer "B.Cu") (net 1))
 (segment (start 144.399 85.598) (end 143.002 86.995) (width 0.508) (layer "B.Cu") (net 1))
 (segment (start 152.4 83.312) (end 150.368 85.344) (width 0.508) (layer "B.Cu") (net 1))
 (segment (start 143.002 86.995) (end 143.002 87.122) (width 0.2) (layer "B.Cu") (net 1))
 (segment (start 153.924 83.312) (end 153.469 83.312) (width 0.2) (layer "B.Cu") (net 1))
 (segment (start 153.924 83.312) (end 152.4 83.312) (width 0.508) (layer "B.Cu") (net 1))
 (segment (start 150.114 85.598) (end 144.399 85.598) (width 0.508) (layer "B.Cu") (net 1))
 (segment (start 158.6865 84.2645) (end 157.734 83.312) (width 0.508) (layer "B.Cu") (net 1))
 (segment (start 150.368 85.344) (end 149.164 84.14) (width 0.508) (layer "B.Cu") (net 1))
 (segment (start 153.469 83.312) (end 153.456 83.299) (width 0.2) (layer "B.Cu") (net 1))
 (segment (start 157.734 83.312) (end 156.464 83.312) (width 0.508) (layer "B.Cu") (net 1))
 (segment (start 150.067 94.949) (end 144.319 94.949) (width 0.508) (layer "B.Cu") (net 10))
 (segment (start 152.146 97.028) (end 150.067 94.949) (width 0.508) (layer "B.Cu") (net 10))
 (segment (start 144.319 91.694) (end 144.319 94.949) (width 0.306) (layer "B.Cu") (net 10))
 (segment (start 155.956 95.758) (end 157.734 95.758) (width 0.508) (layer "B.Cu") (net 11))
 (segment (start 157.734 95.758) (end 157.734 92.249) (width 0.306) (layer "B.Cu") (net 11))
 (segment (start 154.686 97.028) (end 155.956 95.758) (width 0.508) (layer "B.Cu") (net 11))
 (segment (start 157.734 92.249) (end 156.925 91.44) (width 0.508) (layer "B.Cu") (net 11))
 (segment (start 160.782 89.408) (end 158.75 89.408) (width 0.508) (layer "F.Cu") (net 12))
 (via (at 160.782 89.408) (size 1.5) (drill 0.7) (layers "F.Cu" "B.Cu") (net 12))
 (segment (start 160.782 92.456) (end 159.512 93.726) (width 0.508) (layer "B.Cu") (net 12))
 (segment (start 159.512 93.726) (end 158.703 93.726) (width 0.508) (layer "B.Cu") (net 12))
 (segment (start 160.782 89.408) (end 160.782 92.456) (width 0.508) (layer "B.Cu") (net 12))
 (segment (start 154.94 91.948) (end 150.423002 91.948) (width 0.508) (layer "F.Cu") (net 4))
 (segment (start 150.423002 91.948) (end 150.423002 90.424) (width 0.508) (layer "F.Cu") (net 4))
 (segment (start 146.558 91.948) (end 150.423002 91.948) (width 0.508) (layer "F.Cu") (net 4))
 (segment (start 150.423002 91.948) (end 150.423002 90.460998) (width 0.508) (layer "F.Cu") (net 4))
 (segment (start 150.423002 90.460998) (end 150.423002 90.424) (width 0.2) (layer "F.Cu") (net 4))
 (via (at 154.94 91.948) (size 1.5) (drill 0.7) (layers "F.Cu" "B.Cu") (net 4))
 (via (at 146.558 91.948) (size 1.5) (drill 0.7) (layers "F.Cu" "B.Cu") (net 4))
 (segment (start 156.718 93.726) (end 156.878 93.726) (width 0.2) (layer "B.Cu") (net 4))
 (segment (start 146.558 92.202) (end 145.288 93.472) (width 0.508) (layer "B.Cu") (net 4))
 (segment (start 154.94 91.948) (end 156.718 93.726) (width 0.508) (layer "B.Cu") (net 4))
 (segment (start 146.558 91.948) (end 146.558 92.202) (width 0.2) (layer "B.Cu") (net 4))
 (segment (start 145.288 93.472) (end 145.288 93.726) (width 0.2) (layer "B.Cu") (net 4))
 (segment (start 140.97 89.408) (end 142.98 89.408) (width 0.508) (layer "F.Cu") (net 9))
 (via (at 140.97 89.408) (size 1.5) (drill 0.7) (layers "F.Cu" "B.Cu") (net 9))
 (segment (start 140.97 89.408) (end 140.97 92.456) (width 0.508) (layer "B.Cu") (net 9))
 (segment (start 140.97 92.456) (end 142.24 93.726) (width 0.508) (layer "B.Cu") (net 9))
 (segment (start 142.24 93.726) (end 143.463 93.726) (width 0.508) (layer "B.Cu") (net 9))
 (segment (start 153.717 91.139) (end 153.717 93.726) (width 0.508) (layer "B.Cu") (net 14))
 (segment (start 156.7815 88.9508) (end 155.9052 88.9508) (width 0.508) (layer "B.Cu") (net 14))
 (segment (start 155.9052 88.9508) (end 153.717 91.139) (width 0.508) (layer "B.Cu") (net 14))
 (segment (start 157.734 86.868) (end 157.734 89.916) (width 0.508) (layer "B.Cu") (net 13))
 (segment (start 157.734 89.916) (end 158.75 90.932) (width 0.508) (layer "B.Cu") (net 13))
 (segment (start 158.75 90.932) (end 158.75 91.44) (width 0.2) (layer "B.Cu") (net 13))
 (segment (start 144.907 88.011) (end 147.828 90.932) (width 0.508) (layer "B.Cu") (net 15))
 (segment (start 147.828 90.932) (end 147.828 93.726) (width 0.508) (layer "B.Cu") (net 15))
 (segment (start 144.907 87.122) (end 144.907 88.011) (width 0.508) (layer "B.Cu") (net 15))
 (segment (start 142.494 90.424) (end 142.494 91.694) (width 0.508) (layer "B.Cu") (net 16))
 (segment (start 143.764 89.154) (end 142.494 90.424) (width 0.508) (layer "B.Cu") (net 16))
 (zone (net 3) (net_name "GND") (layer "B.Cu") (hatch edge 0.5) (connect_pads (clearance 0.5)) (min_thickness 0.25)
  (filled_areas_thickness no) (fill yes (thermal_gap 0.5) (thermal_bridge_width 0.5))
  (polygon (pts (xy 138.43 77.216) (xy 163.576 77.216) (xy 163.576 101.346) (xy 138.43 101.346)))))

